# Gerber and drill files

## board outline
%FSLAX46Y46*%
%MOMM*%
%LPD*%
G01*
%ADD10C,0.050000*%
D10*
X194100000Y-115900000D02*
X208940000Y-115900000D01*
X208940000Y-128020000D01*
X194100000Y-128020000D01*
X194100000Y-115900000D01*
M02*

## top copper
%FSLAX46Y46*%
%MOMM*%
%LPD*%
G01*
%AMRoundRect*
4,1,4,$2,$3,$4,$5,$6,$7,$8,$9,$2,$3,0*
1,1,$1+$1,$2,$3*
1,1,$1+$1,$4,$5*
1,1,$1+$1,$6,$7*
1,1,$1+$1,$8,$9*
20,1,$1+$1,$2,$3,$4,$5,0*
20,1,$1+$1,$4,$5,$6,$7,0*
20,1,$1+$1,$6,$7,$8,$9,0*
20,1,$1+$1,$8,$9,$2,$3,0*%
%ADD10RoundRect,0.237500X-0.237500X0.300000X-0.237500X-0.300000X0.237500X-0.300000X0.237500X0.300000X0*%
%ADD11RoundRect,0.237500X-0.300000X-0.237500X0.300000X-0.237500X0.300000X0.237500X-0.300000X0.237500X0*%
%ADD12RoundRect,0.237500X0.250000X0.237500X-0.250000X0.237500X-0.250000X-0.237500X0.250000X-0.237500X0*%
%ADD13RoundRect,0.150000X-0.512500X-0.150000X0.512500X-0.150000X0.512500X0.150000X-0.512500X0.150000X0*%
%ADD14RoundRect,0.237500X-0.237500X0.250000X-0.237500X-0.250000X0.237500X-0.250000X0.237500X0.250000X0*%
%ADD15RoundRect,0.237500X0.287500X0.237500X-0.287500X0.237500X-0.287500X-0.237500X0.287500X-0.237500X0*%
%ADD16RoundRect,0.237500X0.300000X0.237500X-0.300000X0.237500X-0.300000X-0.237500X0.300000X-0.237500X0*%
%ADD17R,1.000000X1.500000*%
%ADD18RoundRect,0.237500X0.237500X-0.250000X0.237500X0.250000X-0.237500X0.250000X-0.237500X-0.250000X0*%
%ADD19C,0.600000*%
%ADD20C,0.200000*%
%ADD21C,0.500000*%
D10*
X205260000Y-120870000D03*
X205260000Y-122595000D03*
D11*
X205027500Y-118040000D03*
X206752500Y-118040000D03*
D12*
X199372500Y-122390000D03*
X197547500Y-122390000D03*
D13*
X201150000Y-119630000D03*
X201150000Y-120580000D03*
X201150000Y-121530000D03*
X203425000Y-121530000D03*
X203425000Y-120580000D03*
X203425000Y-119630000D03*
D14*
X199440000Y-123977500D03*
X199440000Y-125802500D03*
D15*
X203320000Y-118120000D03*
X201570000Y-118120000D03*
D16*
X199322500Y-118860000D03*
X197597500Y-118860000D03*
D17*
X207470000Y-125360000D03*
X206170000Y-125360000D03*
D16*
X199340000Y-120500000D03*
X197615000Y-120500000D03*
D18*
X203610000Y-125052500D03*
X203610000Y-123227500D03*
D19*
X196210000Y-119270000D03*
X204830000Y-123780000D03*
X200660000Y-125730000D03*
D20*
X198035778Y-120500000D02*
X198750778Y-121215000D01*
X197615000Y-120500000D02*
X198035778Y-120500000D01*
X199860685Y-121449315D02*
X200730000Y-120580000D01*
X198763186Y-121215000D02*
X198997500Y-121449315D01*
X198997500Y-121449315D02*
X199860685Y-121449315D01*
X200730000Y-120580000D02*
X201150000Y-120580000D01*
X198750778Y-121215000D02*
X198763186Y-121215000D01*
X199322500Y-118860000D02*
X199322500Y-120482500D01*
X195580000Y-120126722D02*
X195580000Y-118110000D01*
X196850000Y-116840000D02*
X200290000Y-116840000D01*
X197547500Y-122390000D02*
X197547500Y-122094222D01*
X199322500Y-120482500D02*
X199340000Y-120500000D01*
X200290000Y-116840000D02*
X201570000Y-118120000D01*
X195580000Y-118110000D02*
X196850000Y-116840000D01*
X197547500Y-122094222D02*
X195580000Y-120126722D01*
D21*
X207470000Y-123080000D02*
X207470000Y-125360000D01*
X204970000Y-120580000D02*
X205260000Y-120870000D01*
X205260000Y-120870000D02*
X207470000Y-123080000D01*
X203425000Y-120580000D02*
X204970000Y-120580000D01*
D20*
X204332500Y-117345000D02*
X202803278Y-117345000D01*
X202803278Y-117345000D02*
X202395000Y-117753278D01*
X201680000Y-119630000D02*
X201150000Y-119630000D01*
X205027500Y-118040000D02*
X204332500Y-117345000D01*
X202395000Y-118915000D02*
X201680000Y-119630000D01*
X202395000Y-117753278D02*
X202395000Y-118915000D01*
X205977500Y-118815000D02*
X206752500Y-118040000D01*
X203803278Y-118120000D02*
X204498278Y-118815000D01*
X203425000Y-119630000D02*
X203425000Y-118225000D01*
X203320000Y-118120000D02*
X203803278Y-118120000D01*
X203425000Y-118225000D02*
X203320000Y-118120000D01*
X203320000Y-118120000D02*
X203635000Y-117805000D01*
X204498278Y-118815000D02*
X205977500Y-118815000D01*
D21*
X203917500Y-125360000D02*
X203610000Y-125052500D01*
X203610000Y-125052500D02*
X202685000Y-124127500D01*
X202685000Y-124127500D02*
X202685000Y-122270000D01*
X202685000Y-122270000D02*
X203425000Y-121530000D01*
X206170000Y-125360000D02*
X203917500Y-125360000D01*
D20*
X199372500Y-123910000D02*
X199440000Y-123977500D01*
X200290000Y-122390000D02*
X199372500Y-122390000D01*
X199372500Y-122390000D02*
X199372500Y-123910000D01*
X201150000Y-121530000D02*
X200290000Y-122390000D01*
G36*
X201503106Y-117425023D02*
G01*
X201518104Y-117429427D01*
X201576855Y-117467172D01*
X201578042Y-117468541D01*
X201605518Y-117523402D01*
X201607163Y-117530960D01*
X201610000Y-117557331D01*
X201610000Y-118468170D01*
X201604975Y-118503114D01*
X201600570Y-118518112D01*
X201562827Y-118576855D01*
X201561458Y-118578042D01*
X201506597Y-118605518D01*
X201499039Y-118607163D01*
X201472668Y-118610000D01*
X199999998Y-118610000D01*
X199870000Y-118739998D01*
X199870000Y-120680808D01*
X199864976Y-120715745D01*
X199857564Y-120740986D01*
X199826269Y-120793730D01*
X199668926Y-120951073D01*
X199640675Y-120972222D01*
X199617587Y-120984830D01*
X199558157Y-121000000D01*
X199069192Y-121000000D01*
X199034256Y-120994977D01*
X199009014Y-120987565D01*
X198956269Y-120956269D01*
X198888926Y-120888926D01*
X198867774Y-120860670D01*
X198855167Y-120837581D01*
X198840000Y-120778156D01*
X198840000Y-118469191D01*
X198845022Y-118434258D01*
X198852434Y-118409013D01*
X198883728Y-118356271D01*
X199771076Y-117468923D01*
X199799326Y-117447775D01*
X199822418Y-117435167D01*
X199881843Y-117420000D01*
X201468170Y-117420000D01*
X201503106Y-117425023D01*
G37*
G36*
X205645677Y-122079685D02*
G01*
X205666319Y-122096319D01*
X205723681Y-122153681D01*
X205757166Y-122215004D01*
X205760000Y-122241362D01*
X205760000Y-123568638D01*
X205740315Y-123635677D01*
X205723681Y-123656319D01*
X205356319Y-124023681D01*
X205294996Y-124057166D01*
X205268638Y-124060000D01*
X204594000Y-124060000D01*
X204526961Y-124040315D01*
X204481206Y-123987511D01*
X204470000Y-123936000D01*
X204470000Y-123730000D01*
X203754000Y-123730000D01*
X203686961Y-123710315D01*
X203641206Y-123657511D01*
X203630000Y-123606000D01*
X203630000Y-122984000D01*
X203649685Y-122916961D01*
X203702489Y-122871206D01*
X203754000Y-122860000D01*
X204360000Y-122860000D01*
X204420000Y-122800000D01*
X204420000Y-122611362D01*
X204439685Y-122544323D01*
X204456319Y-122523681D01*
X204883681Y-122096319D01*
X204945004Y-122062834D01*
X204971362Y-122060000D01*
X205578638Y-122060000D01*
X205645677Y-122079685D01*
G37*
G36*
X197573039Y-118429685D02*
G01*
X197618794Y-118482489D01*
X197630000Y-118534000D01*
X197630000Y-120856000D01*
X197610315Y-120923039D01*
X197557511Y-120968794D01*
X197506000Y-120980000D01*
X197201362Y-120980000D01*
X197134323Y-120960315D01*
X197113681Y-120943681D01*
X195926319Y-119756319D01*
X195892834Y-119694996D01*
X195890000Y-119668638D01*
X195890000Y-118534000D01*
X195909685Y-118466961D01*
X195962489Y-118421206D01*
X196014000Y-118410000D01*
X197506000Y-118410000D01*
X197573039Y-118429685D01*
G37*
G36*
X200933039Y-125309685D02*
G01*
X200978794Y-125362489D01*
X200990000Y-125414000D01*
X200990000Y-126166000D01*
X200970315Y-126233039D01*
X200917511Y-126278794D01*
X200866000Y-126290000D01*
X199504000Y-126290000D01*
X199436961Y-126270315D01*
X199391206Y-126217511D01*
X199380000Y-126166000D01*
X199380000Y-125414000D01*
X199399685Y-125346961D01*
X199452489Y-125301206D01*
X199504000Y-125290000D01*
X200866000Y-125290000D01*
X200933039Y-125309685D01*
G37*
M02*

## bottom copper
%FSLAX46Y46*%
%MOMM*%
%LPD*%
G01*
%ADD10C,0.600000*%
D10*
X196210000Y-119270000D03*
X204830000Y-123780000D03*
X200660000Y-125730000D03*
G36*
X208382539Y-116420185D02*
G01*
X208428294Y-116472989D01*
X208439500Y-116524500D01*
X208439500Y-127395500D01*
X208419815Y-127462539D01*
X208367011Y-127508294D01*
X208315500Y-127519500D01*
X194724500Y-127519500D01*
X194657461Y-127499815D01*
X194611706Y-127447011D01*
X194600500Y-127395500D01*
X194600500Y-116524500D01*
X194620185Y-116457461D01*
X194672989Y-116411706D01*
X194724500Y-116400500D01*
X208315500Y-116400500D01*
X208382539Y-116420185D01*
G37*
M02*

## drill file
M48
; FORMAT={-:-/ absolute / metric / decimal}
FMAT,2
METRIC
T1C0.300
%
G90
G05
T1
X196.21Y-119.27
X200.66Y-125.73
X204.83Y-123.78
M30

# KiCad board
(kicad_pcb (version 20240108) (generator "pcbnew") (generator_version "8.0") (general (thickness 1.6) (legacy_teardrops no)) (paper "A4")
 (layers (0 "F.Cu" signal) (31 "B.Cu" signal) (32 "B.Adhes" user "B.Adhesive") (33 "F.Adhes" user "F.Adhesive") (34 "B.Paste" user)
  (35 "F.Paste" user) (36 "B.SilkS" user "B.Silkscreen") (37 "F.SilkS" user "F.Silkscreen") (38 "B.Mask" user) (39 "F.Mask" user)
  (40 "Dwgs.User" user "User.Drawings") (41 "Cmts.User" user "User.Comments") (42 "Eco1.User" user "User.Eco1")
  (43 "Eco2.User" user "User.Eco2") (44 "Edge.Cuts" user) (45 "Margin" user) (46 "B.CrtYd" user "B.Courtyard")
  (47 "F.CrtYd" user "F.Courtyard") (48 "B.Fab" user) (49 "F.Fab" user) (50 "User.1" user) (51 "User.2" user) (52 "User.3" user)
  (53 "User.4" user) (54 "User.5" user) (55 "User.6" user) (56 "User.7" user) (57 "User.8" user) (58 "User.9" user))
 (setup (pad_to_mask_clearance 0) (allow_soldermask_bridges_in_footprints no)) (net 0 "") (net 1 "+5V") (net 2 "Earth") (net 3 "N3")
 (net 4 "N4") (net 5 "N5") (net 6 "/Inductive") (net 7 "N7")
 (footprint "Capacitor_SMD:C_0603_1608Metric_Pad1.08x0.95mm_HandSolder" (layer "F.Cu") (at 205.26 121.7325 -90)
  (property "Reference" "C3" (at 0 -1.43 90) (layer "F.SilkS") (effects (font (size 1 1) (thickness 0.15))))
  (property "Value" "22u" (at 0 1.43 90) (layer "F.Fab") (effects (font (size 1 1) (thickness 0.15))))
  (pad "1" smd roundrect (at -0.8625 0 270) (size 1.075 0.95) (layers "F.Cu" "F.Paste" "F.Mask") (roundrect_rratio 0.25) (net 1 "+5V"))
  (pad "2" smd roundrect (at 0.8625 0 270) (size 1.075 0.95) (layers "F.Cu" "F.Paste" "F.Mask") (roundrect_rratio 0.25) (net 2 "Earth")))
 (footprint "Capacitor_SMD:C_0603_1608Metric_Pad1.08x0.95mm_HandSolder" (layer "F.Cu") (at 205.89 118.04)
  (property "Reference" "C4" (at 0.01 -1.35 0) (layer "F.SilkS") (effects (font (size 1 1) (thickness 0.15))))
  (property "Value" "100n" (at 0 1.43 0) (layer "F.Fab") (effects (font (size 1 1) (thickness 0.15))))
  (pad "1" smd roundrect (at -0.8625 0) (size 1.075 0.95) (layers "F.Cu" "F.Paste" "F.Mask") (roundrect_rratio 0.25) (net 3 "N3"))
  (pad "2" smd roundrect (at 0.8625 0) (size 1.075 0.95) (layers "F.Cu" "F.Paste" "F.Mask") (roundrect_rratio 0.25) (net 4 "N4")))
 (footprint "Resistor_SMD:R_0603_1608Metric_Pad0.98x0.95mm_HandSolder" (layer "F.Cu") (at 198.46 122.39 180)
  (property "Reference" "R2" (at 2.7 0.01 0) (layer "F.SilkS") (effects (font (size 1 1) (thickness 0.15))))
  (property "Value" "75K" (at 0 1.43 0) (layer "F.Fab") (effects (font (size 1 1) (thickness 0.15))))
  (pad "1" smd roundrect (at -0.9125 0 180) (size 0.975 0.95) (layers "F.Cu" "F.Paste" "F.Mask") (roundrect_rratio 0.25) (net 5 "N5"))
  (pad "2" smd roundrect (at 0.9125 0 180) (size 0.975 0.95) (layers "F.Cu" "F.Paste" "F.Mask") (roundrect_rratio 0.25) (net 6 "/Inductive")))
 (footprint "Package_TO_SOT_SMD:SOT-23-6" (layer "F.Cu") (at 202.2875 120.58)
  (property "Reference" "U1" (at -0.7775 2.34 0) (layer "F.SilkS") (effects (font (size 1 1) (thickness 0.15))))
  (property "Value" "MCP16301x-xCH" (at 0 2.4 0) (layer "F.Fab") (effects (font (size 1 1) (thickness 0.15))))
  (pad "1" smd roundrect (at -1.1375 -0.95) (size 1.325 0.6) (layers "F.Cu" "F.Paste" "F.Mask") (roundrect_rratio 0.25) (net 3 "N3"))
  (pad "2" smd roundrect (at -1.1375 0) (size 1.325 0.6) (layers "F.Cu" "F.Paste" "F.Mask") (roundrect_rratio 0.25) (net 2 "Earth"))
  (pad "3" smd roundrect (at -1.1375 0.95) (size 1.325 0.6) (layers "F.Cu" "F.Paste" "F.Mask") (roundrect_rratio 0.25) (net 5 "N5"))
  (pad "4" smd roundrect (at 1.1375 0.95) (size 1.325 0.6) (layers "F.Cu" "F.Paste" "F.Mask") (roundrect_rratio 0.25) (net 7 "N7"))
  (pad "5" smd roundrect (at 1.1375 0) (size 1.325 0.6) (layers "F.Cu" "F.Paste" "F.Mask") (roundrect_rratio 0.25) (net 1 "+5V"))
  (pad "6" smd roundrect (at 1.1375 -0.95) (size 1.325 0.6) (layers "F.Cu" "F.Paste" "F.Mask") (roundrect_rratio 0.25) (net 4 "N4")))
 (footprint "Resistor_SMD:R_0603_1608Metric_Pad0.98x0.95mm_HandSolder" (layer "F.Cu") (at 199.44 124.89 -90)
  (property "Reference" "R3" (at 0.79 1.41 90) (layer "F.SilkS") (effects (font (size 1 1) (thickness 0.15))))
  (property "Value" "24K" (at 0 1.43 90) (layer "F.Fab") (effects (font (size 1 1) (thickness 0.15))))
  (pad "1" smd roundrect (at -0.9125 0 270) (size 0.975 0.95) (layers "F.Cu" "F.Paste" "F.Mask") (roundrect_rratio 0.25) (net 5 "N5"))
  (pad "2" smd roundrect (at 0.9125 0 270) (size 0.975 0.95) (layers "F.Cu" "F.Paste" "F.Mask") (roundrect_rratio 0.25) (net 2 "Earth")))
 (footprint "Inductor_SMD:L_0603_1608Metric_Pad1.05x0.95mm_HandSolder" (layer "F.Cu") (at 202.445 118.12 180)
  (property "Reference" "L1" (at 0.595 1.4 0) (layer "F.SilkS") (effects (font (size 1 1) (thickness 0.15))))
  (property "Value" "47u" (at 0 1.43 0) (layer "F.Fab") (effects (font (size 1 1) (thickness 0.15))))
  (pad "1" smd roundrect (at -0.875 0 180) (size 1.05 0.95) (layers "F.Cu" "F.Paste" "F.Mask") (roundrect_rratio 0.25) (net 4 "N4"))
  (pad "2" smd roundrect (at 0.875 0 180) (size 1.05 0.95) (layers "F.Cu" "F.Paste" "F.Mask") (roundrect_rratio 0.25) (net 6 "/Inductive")))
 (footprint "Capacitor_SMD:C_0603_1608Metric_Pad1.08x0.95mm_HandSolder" (layer "F.Cu") (at 198.46 118.86 180)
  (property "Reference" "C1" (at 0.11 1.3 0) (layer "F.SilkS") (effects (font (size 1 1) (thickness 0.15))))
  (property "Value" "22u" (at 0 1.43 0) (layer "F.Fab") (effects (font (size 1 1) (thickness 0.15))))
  (pad "1" smd roundrect (at -0.8625 0 180) (size 1.075 0.95) (layers "F.Cu" "F.Paste" "F.Mask") (roundrect_rratio 0.25)
   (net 6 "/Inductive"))
  (pad "2" smd roundrect (at 0.8625 0 180) (size 1.075 0.95) (layers "F.Cu" "F.Paste" "F.Mask") (roundrect_rratio 0.25) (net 2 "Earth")))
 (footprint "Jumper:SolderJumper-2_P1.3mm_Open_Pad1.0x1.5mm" (layer "F.Cu") (at 206.82 125.36 180)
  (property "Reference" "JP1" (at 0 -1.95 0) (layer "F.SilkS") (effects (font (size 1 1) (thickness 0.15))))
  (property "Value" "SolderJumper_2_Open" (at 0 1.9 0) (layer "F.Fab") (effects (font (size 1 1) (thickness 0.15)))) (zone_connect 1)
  (pad "1" smd rect (at -0.65 0 180) (size 1 1.5) (layers "F.Cu" "F.Mask") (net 1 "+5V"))
  (pad "2" smd rect (at 0.65 0 180) (size 1 1.5) (layers "F.Cu" "F.Mask") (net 7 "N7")))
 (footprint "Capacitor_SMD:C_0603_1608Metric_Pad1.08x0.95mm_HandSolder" (layer "F.Cu") (at 198.4775 120.5 180)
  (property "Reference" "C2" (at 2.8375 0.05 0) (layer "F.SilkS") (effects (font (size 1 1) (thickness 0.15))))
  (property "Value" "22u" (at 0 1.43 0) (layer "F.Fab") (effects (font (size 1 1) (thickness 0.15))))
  (pad "1" smd roundrect (at -0.8625 0 180) (size 1.075 0.95) (layers "F.Cu" "F.Paste" "F.Mask") (roundrect_rratio 0.25)
   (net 6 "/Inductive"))
  (pad "2" smd roundrect (at 0.8625 0 180) (size 1.075 0.95) (layers "F.Cu" "F.Paste" "F.Mask") (roundrect_rratio 0.25) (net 2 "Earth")))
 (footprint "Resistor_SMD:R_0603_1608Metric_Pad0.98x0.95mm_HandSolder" (layer "F.Cu") (at 203.61 124.14 90)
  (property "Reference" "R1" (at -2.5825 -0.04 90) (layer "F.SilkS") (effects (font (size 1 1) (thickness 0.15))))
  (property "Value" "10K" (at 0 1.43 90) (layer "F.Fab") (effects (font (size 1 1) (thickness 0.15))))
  (pad "1" smd roundrect (at -0.9125 0 90) (size 0.975 0.95) (layers "F.Cu" "F.Paste" "F.Mask") (roundrect_rratio 0.25) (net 7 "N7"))
  (pad "2" smd roundrect (at 0.9125 0 90) (size 0.975 0.95) (layers "F.Cu" "F.Paste" "F.Mask") (roundrect_rratio 0.25) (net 2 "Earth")))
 (gr_rect (start 194.1 115.9) (end 208.94 128.02) (stroke (width 0.05) (type default)) (fill none) (layer "Edge.Cuts"))
 (segment (start 198.035778 120.5) (end 198.750778 121.215) (width 0.2) (layer "F.Cu") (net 2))
 (segment (start 197.615 120.5) (end 198.035778 120.5) (width 0.2) (layer "F.Cu") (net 2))
 (segment (start 199.860685 121.449315) (end 200.73 120.58) (width 0.2) (layer "F.Cu") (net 2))
 (segment (start 198.763186 121.215) (end 198.9975 121.449315) (width 0.2) (layer "F.Cu") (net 2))
 (segment (start 198.9975 121.449315) (end 199.860685 121.449315) (width 0.2) (layer "F.Cu") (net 2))
 (segment (start 200.73 120.58) (end 201.15 120.58) (width 0.2) (layer "F.Cu") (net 2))
 (segment (start 198.750778 121.215) (end 198.763186 121.215) (width 0.2) (layer "F.Cu") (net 2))
 (via (at 196.21 119.27) (size 0.6) (drill 0.3) (layers "F.Cu" "B.Cu") (free yes) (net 2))
 (via (at 204.83 123.78) (size 0.6) (drill 0.3) (layers "F.Cu" "B.Cu") (free yes) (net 2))
 (via (at 200.66 125.73) (size 0.6) (drill 0.3) (layers "F.Cu" "B.Cu") (free yes) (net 2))
 (segment (start 199.3225 118.86) (end 199.3225 120.4825) (width 0.2) (layer "F.Cu") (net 6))
 (segment (start 195.58 120.126722) (end 195.58 118.11) (width 0.2) (layer "F.Cu") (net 6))
 (segment (start 196.85 116.84) (end 200.29 116.84) (width 0.2) (layer "F.Cu") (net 6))
 (segment (start 197.5475 122.39) (end 197.5475 122.094222) (width 0.2) (layer "F.Cu") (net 6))
 (segment (start 199.3225 120.4825) (end 199.34 120.5) (width 0.2) (layer "F.Cu") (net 6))
 (segment (start 200.29 116.84) (end 201.57 118.12) (width 0.2) (layer "F.Cu") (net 6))
 (segment (start 195.58 118.11) (end 196.85 116.84) (width 0.2) (layer "F.Cu") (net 6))
 (segment (start 197.5475 122.094222) (end 195.58 120.126722) (width 0.2) (layer "F.Cu") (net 6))
 (segment (start 207.47 123.08) (end 207.47 125.36) (width 0.5) (layer "F.Cu") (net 1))
 (segment (start 204.97 120.58) (end 205.26 120.87) (width 0.5) (layer "F.Cu") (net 1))
 (segment (start 205.26 120.87) (end 207.47 123.08) (width 0.5) (layer "F.Cu") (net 1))
 (segment (start 203.425 120.58) (end 204.97 120.58) (width 0.5) (layer "F.Cu") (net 1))
 (segment (start 204.3325 117.345) (end 202.803278 117.345) (width 0.2) (layer "F.Cu") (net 3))
 (segment (start 202.803278 117.345) (end 202.395 117.753278) (width 0.2) (layer "F.Cu") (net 3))
 (segment (start 201.68 119.63) (end 201.15 119.63) (width 0.2) (layer "F.Cu") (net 3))
 (segment (start 205.0275 118.04) (end 204.3325 117.345) (width 0.2) (layer "F.Cu") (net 3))
 (segment (start 202.395 118.915) (end 201.68 119.63) (width 0.2) (layer "F.Cu") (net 3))
 (segment (start 202.395 117.753278) (end 202.395 118.915) (width 0.2) (layer "F.Cu") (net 3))
 (segment (start 205.9775 118.815) (end 206.7525 118.04) (width 0.2) (layer "F.Cu") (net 4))
 (segment (start 203.803278 118.12) (end 204.498278 118.815) (width 0.2) (layer "F.Cu") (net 4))
 (segment (start 203.425 119.63) (end 203.425 118.225) (width 0.2) (layer "F.Cu") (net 4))
 (segment (start 203.32 118.12) (end 203.803278 118.12) (width 0.2) (layer "F.Cu") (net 4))
 (segment (start 203.425 118.225) (end 203.32 118.12) (width 0.2) (layer "F.Cu") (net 4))
 (segment (start 203.32 118.12) (end 203.635 117.805) (width 0.2) (layer "F.Cu") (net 4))
 (segment (start 204.498278 118.815) (end 205.9775 118.815) (width 0.2) (layer "F.Cu") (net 4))
 (segment (start 203.9175 125.36) (end 203.61 125.0525) (width 0.5) (layer "F.Cu") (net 7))
 (segment (start 203.61 125.0525) (end 202.685 124.1275) (width 0.5) (layer "F.Cu") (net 7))
 (segment (start 202.685 124.1275) (end 202.685 122.27) (width 0.5) (layer "F.Cu") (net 7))
 (segment (start 202.685 122.27) (end 203.425 121.53) (width 0.5) (layer "F.Cu") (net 7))
 (segment (start 206.17 125.36) (end 203.9175 125.36) (width 0.5) (layer "F.Cu") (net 7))
 (segment (start 199.3725 123.91) (end 199.44 123.9775) (width 0.2) (layer "F.Cu") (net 5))
 (segment (start 200.29 122.39) (end 199.3725 122.39) (width 0.2) (layer "F.Cu") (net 5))
 (segment (start 199.3725 122.39) (end 199.3725 123.91) (width 0.2) (layer "F.Cu") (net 5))
 (segment (start 201.15 121.53) (end 200.29 122.39) (width 0.2) (layer "F.Cu") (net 5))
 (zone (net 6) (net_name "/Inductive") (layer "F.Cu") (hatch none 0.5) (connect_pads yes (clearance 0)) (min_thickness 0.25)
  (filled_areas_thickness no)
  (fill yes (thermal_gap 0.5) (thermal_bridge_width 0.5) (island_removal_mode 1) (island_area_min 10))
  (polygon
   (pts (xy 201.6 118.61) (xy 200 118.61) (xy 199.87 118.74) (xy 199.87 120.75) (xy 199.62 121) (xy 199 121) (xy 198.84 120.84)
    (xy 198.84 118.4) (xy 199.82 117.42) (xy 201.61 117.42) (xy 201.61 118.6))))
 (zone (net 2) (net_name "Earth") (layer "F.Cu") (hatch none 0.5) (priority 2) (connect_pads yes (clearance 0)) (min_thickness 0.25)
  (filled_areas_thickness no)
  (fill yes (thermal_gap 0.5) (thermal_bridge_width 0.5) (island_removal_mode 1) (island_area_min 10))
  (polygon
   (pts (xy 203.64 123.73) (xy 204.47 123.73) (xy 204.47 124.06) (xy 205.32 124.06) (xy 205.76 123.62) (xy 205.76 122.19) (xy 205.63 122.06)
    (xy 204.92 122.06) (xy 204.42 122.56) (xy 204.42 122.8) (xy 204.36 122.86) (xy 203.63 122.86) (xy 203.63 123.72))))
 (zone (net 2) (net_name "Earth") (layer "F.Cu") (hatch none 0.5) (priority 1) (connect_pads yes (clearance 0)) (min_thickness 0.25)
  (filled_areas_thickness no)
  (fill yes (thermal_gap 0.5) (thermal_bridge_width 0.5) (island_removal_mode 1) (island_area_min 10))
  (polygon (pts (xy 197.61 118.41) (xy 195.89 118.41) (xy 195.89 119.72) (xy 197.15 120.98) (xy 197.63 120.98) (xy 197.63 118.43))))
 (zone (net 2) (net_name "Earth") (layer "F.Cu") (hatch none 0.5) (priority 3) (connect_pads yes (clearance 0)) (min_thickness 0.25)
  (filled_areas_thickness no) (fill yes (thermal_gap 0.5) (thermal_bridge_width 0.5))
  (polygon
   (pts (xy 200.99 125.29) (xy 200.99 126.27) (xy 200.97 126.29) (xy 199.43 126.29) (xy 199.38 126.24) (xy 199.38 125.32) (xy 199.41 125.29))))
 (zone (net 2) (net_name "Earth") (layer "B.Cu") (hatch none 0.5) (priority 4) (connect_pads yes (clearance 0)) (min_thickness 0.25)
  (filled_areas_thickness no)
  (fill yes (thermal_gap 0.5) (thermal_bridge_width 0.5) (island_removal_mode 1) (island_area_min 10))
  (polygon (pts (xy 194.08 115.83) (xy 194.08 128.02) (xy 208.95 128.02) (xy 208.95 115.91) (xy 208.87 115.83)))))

